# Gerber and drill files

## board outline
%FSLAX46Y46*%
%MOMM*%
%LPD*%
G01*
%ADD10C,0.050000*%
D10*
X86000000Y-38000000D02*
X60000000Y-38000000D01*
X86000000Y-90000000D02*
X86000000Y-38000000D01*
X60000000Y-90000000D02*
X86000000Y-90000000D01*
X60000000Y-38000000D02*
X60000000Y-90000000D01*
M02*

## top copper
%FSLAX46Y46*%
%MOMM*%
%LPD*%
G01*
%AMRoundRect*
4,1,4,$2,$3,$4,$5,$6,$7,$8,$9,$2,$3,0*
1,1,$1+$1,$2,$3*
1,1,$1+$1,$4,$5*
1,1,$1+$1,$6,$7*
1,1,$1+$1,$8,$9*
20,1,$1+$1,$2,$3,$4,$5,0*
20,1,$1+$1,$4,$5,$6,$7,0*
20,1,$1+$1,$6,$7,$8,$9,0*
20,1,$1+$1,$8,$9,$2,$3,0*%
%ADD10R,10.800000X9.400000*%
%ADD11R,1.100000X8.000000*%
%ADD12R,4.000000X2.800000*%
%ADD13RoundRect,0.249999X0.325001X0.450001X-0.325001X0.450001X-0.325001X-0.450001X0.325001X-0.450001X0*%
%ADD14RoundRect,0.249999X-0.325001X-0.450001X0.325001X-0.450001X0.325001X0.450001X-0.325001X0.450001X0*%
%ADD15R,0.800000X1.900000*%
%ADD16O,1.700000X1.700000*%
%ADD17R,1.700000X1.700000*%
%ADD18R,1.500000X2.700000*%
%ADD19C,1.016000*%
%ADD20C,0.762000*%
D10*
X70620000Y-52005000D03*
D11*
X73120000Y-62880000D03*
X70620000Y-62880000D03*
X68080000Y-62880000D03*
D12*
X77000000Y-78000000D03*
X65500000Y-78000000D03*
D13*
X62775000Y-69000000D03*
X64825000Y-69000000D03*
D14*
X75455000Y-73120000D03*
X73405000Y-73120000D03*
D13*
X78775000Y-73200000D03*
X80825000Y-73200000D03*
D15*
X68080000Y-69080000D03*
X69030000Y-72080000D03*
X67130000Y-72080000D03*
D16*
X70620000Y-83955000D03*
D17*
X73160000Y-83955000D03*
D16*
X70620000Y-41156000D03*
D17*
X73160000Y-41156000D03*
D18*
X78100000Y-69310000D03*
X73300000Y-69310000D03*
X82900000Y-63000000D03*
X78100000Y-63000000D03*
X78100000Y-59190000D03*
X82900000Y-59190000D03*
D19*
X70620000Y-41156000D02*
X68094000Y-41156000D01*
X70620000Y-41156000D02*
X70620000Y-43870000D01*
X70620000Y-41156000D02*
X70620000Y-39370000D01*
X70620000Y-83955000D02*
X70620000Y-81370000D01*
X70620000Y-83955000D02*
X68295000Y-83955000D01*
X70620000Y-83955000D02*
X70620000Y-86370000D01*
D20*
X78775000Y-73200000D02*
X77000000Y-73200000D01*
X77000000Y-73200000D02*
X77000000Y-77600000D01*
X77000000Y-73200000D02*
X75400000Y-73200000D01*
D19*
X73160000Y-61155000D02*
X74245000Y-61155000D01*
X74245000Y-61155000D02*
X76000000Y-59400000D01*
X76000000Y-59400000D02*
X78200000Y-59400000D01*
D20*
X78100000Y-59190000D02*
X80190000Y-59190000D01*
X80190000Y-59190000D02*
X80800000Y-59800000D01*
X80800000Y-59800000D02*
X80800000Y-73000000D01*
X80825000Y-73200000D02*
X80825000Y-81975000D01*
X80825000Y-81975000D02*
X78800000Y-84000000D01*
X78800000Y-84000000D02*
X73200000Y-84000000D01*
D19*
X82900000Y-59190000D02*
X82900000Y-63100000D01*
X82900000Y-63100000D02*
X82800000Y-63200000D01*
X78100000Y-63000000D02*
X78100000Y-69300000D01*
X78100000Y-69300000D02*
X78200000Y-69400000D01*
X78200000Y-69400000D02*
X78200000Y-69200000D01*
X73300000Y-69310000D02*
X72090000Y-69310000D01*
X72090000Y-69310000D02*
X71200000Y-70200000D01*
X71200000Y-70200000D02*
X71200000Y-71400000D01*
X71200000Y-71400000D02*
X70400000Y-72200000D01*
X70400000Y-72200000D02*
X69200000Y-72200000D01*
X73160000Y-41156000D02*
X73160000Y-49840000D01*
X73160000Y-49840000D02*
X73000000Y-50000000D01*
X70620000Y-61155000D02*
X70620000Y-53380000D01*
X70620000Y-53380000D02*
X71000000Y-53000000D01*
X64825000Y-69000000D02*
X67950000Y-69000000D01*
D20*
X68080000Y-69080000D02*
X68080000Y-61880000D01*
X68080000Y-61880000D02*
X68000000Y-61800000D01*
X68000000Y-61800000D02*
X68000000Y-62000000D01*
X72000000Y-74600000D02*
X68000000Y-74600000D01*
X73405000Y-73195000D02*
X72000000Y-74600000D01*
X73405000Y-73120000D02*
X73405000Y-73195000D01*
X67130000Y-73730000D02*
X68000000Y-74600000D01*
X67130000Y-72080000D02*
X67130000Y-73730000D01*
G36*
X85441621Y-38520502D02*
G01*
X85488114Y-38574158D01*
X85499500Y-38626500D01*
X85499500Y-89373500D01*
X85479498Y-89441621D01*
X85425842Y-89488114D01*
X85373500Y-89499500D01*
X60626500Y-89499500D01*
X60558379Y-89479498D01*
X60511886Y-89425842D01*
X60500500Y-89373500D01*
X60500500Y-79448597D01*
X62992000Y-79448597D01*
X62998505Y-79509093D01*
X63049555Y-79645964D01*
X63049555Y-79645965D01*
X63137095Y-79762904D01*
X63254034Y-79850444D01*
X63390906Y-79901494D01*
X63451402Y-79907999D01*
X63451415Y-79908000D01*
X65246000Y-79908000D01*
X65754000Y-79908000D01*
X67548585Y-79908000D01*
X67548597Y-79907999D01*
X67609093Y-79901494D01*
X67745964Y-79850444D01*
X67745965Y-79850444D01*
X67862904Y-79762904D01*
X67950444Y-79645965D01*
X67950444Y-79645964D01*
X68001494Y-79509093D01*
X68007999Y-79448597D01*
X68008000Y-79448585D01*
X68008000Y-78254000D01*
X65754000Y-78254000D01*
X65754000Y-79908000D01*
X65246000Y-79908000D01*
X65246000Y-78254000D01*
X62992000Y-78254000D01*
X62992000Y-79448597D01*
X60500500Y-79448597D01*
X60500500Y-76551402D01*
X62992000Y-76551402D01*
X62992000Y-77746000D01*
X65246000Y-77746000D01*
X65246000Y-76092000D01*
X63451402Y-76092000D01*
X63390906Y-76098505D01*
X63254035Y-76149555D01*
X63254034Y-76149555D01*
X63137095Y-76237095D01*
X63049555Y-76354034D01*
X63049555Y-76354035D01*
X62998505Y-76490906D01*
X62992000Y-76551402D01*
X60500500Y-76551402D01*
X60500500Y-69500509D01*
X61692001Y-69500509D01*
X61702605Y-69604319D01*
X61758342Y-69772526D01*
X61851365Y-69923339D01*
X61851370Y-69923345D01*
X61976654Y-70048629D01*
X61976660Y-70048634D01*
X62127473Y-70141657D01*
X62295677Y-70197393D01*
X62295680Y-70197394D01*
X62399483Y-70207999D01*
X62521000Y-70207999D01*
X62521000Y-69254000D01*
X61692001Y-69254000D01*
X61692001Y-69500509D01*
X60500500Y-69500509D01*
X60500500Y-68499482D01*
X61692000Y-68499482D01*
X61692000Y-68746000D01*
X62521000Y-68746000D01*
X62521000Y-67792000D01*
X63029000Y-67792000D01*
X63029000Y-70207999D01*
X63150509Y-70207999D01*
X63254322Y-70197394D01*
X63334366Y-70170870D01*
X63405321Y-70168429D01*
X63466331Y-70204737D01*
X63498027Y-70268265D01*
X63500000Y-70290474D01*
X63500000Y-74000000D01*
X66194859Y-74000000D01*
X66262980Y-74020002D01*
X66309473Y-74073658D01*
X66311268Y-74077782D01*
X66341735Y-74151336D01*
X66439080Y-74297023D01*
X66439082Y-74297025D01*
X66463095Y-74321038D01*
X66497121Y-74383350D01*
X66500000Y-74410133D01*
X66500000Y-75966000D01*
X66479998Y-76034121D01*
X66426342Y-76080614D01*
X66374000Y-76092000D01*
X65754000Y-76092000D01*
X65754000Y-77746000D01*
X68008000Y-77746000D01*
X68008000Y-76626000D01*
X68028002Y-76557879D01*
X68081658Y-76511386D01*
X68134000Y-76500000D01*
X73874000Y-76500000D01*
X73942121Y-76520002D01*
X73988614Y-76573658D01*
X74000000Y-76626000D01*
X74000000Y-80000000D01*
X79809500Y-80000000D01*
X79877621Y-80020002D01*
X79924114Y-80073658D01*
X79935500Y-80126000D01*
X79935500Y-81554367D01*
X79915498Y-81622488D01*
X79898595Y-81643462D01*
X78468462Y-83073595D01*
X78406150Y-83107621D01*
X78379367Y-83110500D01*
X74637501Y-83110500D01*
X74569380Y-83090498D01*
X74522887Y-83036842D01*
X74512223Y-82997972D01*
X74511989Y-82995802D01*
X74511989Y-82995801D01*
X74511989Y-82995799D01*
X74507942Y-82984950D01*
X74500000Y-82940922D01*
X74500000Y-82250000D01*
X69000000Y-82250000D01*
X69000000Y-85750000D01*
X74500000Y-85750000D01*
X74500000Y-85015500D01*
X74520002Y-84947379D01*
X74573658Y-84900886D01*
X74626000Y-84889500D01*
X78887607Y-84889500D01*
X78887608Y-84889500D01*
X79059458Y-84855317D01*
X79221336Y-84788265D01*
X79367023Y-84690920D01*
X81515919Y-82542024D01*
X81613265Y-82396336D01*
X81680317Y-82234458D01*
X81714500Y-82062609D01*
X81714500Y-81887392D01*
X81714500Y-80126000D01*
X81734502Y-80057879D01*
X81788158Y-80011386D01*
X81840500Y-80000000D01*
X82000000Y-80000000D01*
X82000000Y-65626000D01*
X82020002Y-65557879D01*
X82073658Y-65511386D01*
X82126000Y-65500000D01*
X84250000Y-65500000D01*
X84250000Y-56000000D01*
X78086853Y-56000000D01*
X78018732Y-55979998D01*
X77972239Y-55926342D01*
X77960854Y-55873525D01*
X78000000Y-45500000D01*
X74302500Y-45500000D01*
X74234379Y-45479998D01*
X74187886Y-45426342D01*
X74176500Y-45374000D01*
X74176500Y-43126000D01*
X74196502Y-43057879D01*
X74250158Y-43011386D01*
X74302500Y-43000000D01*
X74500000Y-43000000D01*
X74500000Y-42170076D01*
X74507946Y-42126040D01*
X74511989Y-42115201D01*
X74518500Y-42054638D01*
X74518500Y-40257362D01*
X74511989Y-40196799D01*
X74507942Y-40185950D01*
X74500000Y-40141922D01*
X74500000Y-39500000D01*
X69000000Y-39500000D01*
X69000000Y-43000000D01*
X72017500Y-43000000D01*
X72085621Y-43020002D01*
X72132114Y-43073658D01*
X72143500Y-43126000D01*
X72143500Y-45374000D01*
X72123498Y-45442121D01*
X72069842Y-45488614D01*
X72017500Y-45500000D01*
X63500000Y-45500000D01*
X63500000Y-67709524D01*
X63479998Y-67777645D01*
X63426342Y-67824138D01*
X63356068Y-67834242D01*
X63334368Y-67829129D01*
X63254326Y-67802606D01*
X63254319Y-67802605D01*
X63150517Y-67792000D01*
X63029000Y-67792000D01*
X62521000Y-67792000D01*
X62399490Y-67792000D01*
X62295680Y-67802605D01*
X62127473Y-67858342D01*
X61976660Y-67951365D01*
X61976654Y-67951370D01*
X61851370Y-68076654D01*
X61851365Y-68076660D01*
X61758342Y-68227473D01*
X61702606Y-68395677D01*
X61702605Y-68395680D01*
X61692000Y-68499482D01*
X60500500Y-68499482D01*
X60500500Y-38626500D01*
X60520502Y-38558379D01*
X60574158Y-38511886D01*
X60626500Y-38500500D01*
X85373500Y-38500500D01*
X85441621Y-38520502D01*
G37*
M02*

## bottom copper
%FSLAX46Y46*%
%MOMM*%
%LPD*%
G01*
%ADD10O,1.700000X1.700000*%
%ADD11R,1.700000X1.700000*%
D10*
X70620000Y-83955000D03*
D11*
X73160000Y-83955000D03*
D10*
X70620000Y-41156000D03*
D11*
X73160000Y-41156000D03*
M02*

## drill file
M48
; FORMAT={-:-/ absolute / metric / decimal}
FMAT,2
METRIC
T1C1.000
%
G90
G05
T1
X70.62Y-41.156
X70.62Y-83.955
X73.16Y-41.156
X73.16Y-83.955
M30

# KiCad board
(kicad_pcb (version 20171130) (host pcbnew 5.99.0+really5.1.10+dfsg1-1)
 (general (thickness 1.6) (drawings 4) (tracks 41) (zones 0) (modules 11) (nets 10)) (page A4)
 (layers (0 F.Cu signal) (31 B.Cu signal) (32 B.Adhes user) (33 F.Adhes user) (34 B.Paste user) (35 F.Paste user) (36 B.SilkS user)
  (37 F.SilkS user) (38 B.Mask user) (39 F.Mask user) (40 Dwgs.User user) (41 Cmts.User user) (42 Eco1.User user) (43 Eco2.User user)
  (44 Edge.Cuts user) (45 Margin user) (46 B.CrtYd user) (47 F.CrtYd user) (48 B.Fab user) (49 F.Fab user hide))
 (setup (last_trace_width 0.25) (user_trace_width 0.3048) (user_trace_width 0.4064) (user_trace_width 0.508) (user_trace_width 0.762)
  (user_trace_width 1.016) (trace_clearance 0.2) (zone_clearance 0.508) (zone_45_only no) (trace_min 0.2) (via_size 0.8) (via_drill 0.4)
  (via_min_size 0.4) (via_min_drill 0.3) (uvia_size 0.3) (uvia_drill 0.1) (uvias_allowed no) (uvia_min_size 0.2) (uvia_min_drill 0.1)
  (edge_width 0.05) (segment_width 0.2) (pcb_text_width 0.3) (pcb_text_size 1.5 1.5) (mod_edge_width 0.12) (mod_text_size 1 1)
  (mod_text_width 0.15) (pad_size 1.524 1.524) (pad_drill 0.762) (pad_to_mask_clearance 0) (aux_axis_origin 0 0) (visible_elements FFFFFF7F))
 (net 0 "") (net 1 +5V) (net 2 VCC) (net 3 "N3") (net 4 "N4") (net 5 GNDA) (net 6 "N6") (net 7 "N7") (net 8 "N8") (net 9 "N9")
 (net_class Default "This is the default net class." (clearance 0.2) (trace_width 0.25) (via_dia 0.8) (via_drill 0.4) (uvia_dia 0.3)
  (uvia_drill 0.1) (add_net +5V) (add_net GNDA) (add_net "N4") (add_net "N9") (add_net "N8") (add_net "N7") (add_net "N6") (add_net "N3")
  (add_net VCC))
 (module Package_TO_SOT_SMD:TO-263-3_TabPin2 (layer F.Cu) (at 70.62 55.38 90)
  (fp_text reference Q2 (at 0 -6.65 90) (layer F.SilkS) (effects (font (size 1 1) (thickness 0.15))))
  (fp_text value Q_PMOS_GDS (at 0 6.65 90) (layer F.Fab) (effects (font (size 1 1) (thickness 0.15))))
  (pad "" smd rect (at 0.95 2.775 90) (size 4.55 5.25) (layers F.Paste))
  (pad "" smd rect (at 5.8 -2.775 90) (size 4.55 5.25) (layers F.Paste))
  (pad "" smd rect (at 0.95 -2.775 90) (size 4.55 5.25) (layers F.Paste))
  (pad "" smd rect (at 5.8 2.775 90) (size 4.55 5.25) (layers F.Paste))
  (pad 2 smd rect (at 3.375 0 90) (size 9.4 10.8) (layers F.Cu F.Mask) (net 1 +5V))
  (pad 3 smd rect (at -7.5 2.5 90) (size 8 1.1) (layers F.Cu F.Paste F.Mask) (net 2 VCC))
  (pad 2 smd rect (at -7.5 0 90) (size 8 1.1) (layers F.Cu F.Paste F.Mask) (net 1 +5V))
  (pad 1 smd rect (at -7.5 -2.54 90) (size 8 1.1) (layers F.Cu F.Paste F.Mask) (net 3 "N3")))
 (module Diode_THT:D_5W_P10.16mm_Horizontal (layer F.Cu) (at 77 78 180)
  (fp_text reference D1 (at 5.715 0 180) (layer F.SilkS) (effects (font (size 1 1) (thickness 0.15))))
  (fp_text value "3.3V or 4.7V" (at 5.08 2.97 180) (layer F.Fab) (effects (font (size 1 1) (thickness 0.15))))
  (pad 1 smd rect (at 0 0 180) (size 4 2.8) (layers F.Cu F.Paste F.Mask) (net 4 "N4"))
  (pad 2 smd rect (at 11.5 0 180) (size 4 2.8) (layers F.Cu F.Paste F.Mask) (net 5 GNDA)))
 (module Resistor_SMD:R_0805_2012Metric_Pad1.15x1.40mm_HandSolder (layer F.Cu) (at 63.8 69 180)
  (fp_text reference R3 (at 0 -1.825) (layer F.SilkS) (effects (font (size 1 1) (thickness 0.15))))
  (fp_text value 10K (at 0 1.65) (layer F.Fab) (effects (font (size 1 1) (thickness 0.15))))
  (pad 2 smd roundrect (at 1.025 0 180) (size 1.15 1.4) (layers F.Cu F.Paste F.Mask) (roundrect_rratio 0.2173904347826087) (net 5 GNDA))
  (pad 1 smd roundrect (at -1.025 0 180) (size 1.15 1.4) (layers F.Cu F.Paste F.Mask) (roundrect_rratio 0.2173904347826087) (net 3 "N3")))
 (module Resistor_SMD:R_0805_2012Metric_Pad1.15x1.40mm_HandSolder (layer F.Cu) (at 74.43 73.12)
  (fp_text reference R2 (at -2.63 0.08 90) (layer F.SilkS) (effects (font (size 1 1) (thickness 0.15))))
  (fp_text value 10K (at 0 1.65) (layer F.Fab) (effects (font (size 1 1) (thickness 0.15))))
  (pad 2 smd roundrect (at 1.025 0) (size 1.15 1.4) (layers F.Cu F.Paste F.Mask) (roundrect_rratio 0.2173904347826087) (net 4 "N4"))
  (pad 1 smd roundrect (at -1.025 0) (size 1.15 1.4) (layers F.Cu F.Paste F.Mask) (roundrect_rratio 0.2173904347826087) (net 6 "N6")))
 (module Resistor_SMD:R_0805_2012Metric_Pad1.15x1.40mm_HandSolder (layer F.Cu) (at 79.8 73.2 180)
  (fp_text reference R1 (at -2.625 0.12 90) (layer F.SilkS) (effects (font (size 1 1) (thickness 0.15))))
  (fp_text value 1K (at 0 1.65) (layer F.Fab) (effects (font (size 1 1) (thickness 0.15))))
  (pad 2 smd roundrect (at 1.025 0 180) (size 1.15 1.4) (layers F.Cu F.Paste F.Mask) (roundrect_rratio 0.2173904347826087) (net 4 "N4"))
  (pad 1 smd roundrect (at -1.025 0 180) (size 1.15 1.4) (layers F.Cu F.Paste F.Mask) (roundrect_rratio 0.2173904347826087) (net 2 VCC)))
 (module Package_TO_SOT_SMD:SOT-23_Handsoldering (layer F.Cu) (at 68.08 70.58 90)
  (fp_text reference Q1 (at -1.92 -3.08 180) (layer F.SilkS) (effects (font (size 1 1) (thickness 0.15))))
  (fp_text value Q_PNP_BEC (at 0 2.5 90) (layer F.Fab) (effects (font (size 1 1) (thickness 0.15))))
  (pad 3 smd rect (at 1.5 0 90) (size 1.9 0.8) (layers F.Cu F.Paste F.Mask) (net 3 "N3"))
  (pad 2 smd rect (at -1.5 0.95 90) (size 1.9 0.8) (layers F.Cu F.Paste F.Mask) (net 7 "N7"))
  (pad 1 smd rect (at -1.5 -0.95 90) (size 1.9 0.8) (layers F.Cu F.Paste F.Mask) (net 6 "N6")))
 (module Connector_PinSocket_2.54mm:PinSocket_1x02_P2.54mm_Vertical (layer F.Cu) (at 73.16 83.955 270)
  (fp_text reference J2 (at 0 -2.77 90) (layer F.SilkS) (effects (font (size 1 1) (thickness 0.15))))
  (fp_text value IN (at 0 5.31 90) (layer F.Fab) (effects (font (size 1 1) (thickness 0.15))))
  (pad 2 thru_hole oval (at 0 2.54 270) (size 1.7 1.7) (drill 1) (layers *.Cu *.Mask) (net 5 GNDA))
  (pad 1 thru_hole rect (at 0 0 270) (size 1.7 1.7) (drill 1) (layers *.Cu *.Mask) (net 2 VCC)))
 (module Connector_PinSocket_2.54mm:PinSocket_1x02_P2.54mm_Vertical (layer F.Cu) (at 73.16 41.156 270)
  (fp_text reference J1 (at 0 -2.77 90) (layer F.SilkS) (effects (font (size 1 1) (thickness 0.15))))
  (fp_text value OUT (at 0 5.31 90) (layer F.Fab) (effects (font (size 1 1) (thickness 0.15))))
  (pad 2 thru_hole oval (at 0 2.54 270) (size 1.7 1.7) (drill 1) (layers *.Cu *.Mask) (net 5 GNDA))
  (pad 1 thru_hole rect (at 0 0 270) (size 1.7 1.7) (drill 1) (layers *.Cu *.Mask) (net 1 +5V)))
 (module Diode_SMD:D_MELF (layer F.Cu) (at 75.7 69.31)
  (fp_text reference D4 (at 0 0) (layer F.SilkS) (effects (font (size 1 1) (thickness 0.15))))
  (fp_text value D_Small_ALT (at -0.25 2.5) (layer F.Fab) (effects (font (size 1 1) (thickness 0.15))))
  (pad 2 smd rect (at 2.4 0) (size 1.5 2.7) (layers F.Cu F.Paste F.Mask) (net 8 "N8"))
  (pad 1 smd rect (at -2.4 0) (size 1.5 2.7) (layers F.Cu F.Paste F.Mask) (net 7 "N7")))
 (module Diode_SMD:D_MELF (layer F.Cu) (at 80.5 63)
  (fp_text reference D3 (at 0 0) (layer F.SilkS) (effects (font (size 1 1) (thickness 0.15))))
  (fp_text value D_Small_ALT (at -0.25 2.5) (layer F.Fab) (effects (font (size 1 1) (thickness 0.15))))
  (pad 2 smd rect (at 2.4 0) (size 1.5 2.7) (layers F.Cu F.Paste F.Mask) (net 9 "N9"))
  (pad 1 smd rect (at -2.4 0) (size 1.5 2.7) (layers F.Cu F.Paste F.Mask) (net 8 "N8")))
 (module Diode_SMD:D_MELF (layer F.Cu) (at 80.5 59.19 180)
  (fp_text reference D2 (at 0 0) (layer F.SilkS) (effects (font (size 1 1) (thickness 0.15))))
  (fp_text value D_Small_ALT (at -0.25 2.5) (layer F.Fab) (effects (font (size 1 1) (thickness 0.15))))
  (pad 2 smd rect (at 2.4 0 180) (size 1.5 2.7) (layers F.Cu F.Paste F.Mask) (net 2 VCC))
  (pad 1 smd rect (at -2.4 0 180) (size 1.5 2.7) (layers F.Cu F.Paste F.Mask) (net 9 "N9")))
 (gr_line (start 86 38) (end 60 38) (layer Edge.Cuts) (width 0.05))
 (gr_line (start 86 90) (end 86 38) (layer Edge.Cuts) (width 0.05))
 (gr_line (start 60 90) (end 86 90) (layer Edge.Cuts) (width 0.05))
 (gr_line (start 60 38) (end 60 90) (layer Edge.Cuts) (width 0.05))
 (segment (start 70.62 41.156) (end 68.094 41.156) (width 1.016) (layer F.Cu) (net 5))
 (segment (start 70.62 41.156) (end 70.62 43.87) (width 1.016) (layer F.Cu) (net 5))
 (segment (start 70.62 41.156) (end 70.62 39.37) (width 1.016) (layer F.Cu) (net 5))
 (segment (start 70.62 83.955) (end 70.62 81.37) (width 1.016) (layer F.Cu) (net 5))
 (segment (start 70.62 83.955) (end 68.295 83.955) (width 1.016) (layer F.Cu) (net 5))
 (segment (start 70.62 83.955) (end 70.62 86.37) (width 1.016) (layer F.Cu) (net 5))
 (segment (start 78.775 73.2) (end 77 73.2) (width 0.762) (layer F.Cu) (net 4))
 (segment (start 77 73.2) (end 77 77.6) (width 0.762) (layer F.Cu) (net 4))
 (segment (start 77 73.2) (end 75.4 73.2) (width 0.762) (layer F.Cu) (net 4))
 (segment (start 73.16 61.155) (end 74.245 61.155) (width 1.016) (layer F.Cu) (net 2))
 (segment (start 74.245 61.155) (end 76 59.4) (width 1.016) (layer F.Cu) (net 2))
 (segment (start 76 59.4) (end 78.2 59.4) (width 1.016) (layer F.Cu) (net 2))
 (segment (start 78.1 59.19) (end 80.19 59.19) (width 0.762) (layer F.Cu) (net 2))
 (segment (start 80.19 59.19) (end 80.8 59.8) (width 0.762) (layer F.Cu) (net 2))
 (segment (start 80.8 59.8) (end 80.8 73) (width 0.762) (layer F.Cu) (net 2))
 (segment (start 80.825 73.2) (end 80.825 81.975) (width 0.762) (layer F.Cu) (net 2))
 (segment (start 80.825 81.975) (end 78.8 84) (width 0.762) (layer F.Cu) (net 2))
 (segment (start 78.8 84) (end 73.2 84) (width 0.762) (layer F.Cu) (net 2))
 (segment (start 82.9 59.19) (end 82.9 63.1) (width 1.016) (layer F.Cu) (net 9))
 (segment (start 82.9 63.1) (end 82.8 63.2) (width 1.016) (layer F.Cu) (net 9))
 (segment (start 78.1 63) (end 78.1 69.3) (width 1.016) (layer F.Cu) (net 8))
 (segment (start 78.1 69.3) (end 78.2 69.4) (width 1.016) (layer F.Cu) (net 8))
 (segment (start 78.2 69.4) (end 78.2 69.2) (width 1.016) (layer F.Cu) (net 8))
 (segment (start 73.3 69.31) (end 72.09 69.31) (width 1.016) (layer F.Cu) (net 7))
 (segment (start 72.09 69.31) (end 71.2 70.2) (width 1.016) (layer F.Cu) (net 7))
 (segment (start 71.2 70.2) (end 71.2 71.4) (width 1.016) (layer F.Cu) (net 7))
 (segment (start 71.2 71.4) (end 70.4 72.2) (width 1.016) (layer F.Cu) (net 7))
 (segment (start 70.4 72.2) (end 69.2 72.2) (width 1.016) (layer F.Cu) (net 7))
 (segment (start 73.16 41.156) (end 73.16 49.84) (width 1.016) (layer F.Cu) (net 1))
 (segment (start 73.16 49.84) (end 73 50) (width 1.016) (layer F.Cu) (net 1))
 (segment (start 70.62 61.155) (end 70.62 53.38) (width 1.016) (layer F.Cu) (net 1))
 (segment (start 70.62 53.38) (end 71 53) (width 1.016) (layer F.Cu) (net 1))
 (segment (start 64.825 69) (end 67.95 69) (width 1.016) (layer F.Cu) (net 3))
 (segment (start 68.08 69.08) (end 68.08 61.88) (width 0.762) (layer F.Cu) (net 3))
 (segment (start 68.08 61.88) (end 68 61.8) (width 0.762) (layer F.Cu) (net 3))
 (segment (start 68 61.8) (end 68 62) (width 0.762) (layer F.Cu) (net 3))
 (segment (start 72 74.6) (end 68 74.6) (width 0.762) (layer F.Cu) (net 6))
 (segment (start 73.405 73.195) (end 72 74.6) (width 0.762) (layer F.Cu) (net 6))
 (segment (start 73.405 73.12) (end 73.405 73.195) (width 0.762) (layer F.Cu) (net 6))
 (segment (start 67.13 73.73) (end 68 74.6) (width 0.762) (layer F.Cu) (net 6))
 (segment (start 67.13 72.08) (end 67.13 73.73) (width 0.762) (layer F.Cu) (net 6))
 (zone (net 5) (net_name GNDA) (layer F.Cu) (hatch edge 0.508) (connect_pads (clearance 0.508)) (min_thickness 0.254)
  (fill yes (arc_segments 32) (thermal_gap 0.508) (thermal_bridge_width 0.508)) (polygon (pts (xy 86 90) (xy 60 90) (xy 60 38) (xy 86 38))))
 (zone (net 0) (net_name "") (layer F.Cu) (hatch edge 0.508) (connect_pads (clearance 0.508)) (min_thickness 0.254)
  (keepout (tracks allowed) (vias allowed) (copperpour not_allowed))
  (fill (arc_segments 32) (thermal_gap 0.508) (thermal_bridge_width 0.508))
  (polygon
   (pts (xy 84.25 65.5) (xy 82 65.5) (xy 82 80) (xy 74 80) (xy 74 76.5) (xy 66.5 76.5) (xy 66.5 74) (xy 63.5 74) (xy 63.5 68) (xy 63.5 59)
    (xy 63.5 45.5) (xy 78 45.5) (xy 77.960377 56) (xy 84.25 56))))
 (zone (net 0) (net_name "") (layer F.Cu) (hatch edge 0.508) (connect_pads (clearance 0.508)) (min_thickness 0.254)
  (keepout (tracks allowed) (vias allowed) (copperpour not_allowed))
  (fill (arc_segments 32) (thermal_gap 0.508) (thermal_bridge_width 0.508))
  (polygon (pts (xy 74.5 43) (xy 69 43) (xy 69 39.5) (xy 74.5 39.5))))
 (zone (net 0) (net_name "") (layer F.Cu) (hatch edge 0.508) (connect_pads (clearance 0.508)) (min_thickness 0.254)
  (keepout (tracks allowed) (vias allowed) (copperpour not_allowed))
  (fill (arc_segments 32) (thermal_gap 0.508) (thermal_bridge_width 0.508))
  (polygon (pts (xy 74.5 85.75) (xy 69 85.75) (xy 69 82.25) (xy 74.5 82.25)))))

